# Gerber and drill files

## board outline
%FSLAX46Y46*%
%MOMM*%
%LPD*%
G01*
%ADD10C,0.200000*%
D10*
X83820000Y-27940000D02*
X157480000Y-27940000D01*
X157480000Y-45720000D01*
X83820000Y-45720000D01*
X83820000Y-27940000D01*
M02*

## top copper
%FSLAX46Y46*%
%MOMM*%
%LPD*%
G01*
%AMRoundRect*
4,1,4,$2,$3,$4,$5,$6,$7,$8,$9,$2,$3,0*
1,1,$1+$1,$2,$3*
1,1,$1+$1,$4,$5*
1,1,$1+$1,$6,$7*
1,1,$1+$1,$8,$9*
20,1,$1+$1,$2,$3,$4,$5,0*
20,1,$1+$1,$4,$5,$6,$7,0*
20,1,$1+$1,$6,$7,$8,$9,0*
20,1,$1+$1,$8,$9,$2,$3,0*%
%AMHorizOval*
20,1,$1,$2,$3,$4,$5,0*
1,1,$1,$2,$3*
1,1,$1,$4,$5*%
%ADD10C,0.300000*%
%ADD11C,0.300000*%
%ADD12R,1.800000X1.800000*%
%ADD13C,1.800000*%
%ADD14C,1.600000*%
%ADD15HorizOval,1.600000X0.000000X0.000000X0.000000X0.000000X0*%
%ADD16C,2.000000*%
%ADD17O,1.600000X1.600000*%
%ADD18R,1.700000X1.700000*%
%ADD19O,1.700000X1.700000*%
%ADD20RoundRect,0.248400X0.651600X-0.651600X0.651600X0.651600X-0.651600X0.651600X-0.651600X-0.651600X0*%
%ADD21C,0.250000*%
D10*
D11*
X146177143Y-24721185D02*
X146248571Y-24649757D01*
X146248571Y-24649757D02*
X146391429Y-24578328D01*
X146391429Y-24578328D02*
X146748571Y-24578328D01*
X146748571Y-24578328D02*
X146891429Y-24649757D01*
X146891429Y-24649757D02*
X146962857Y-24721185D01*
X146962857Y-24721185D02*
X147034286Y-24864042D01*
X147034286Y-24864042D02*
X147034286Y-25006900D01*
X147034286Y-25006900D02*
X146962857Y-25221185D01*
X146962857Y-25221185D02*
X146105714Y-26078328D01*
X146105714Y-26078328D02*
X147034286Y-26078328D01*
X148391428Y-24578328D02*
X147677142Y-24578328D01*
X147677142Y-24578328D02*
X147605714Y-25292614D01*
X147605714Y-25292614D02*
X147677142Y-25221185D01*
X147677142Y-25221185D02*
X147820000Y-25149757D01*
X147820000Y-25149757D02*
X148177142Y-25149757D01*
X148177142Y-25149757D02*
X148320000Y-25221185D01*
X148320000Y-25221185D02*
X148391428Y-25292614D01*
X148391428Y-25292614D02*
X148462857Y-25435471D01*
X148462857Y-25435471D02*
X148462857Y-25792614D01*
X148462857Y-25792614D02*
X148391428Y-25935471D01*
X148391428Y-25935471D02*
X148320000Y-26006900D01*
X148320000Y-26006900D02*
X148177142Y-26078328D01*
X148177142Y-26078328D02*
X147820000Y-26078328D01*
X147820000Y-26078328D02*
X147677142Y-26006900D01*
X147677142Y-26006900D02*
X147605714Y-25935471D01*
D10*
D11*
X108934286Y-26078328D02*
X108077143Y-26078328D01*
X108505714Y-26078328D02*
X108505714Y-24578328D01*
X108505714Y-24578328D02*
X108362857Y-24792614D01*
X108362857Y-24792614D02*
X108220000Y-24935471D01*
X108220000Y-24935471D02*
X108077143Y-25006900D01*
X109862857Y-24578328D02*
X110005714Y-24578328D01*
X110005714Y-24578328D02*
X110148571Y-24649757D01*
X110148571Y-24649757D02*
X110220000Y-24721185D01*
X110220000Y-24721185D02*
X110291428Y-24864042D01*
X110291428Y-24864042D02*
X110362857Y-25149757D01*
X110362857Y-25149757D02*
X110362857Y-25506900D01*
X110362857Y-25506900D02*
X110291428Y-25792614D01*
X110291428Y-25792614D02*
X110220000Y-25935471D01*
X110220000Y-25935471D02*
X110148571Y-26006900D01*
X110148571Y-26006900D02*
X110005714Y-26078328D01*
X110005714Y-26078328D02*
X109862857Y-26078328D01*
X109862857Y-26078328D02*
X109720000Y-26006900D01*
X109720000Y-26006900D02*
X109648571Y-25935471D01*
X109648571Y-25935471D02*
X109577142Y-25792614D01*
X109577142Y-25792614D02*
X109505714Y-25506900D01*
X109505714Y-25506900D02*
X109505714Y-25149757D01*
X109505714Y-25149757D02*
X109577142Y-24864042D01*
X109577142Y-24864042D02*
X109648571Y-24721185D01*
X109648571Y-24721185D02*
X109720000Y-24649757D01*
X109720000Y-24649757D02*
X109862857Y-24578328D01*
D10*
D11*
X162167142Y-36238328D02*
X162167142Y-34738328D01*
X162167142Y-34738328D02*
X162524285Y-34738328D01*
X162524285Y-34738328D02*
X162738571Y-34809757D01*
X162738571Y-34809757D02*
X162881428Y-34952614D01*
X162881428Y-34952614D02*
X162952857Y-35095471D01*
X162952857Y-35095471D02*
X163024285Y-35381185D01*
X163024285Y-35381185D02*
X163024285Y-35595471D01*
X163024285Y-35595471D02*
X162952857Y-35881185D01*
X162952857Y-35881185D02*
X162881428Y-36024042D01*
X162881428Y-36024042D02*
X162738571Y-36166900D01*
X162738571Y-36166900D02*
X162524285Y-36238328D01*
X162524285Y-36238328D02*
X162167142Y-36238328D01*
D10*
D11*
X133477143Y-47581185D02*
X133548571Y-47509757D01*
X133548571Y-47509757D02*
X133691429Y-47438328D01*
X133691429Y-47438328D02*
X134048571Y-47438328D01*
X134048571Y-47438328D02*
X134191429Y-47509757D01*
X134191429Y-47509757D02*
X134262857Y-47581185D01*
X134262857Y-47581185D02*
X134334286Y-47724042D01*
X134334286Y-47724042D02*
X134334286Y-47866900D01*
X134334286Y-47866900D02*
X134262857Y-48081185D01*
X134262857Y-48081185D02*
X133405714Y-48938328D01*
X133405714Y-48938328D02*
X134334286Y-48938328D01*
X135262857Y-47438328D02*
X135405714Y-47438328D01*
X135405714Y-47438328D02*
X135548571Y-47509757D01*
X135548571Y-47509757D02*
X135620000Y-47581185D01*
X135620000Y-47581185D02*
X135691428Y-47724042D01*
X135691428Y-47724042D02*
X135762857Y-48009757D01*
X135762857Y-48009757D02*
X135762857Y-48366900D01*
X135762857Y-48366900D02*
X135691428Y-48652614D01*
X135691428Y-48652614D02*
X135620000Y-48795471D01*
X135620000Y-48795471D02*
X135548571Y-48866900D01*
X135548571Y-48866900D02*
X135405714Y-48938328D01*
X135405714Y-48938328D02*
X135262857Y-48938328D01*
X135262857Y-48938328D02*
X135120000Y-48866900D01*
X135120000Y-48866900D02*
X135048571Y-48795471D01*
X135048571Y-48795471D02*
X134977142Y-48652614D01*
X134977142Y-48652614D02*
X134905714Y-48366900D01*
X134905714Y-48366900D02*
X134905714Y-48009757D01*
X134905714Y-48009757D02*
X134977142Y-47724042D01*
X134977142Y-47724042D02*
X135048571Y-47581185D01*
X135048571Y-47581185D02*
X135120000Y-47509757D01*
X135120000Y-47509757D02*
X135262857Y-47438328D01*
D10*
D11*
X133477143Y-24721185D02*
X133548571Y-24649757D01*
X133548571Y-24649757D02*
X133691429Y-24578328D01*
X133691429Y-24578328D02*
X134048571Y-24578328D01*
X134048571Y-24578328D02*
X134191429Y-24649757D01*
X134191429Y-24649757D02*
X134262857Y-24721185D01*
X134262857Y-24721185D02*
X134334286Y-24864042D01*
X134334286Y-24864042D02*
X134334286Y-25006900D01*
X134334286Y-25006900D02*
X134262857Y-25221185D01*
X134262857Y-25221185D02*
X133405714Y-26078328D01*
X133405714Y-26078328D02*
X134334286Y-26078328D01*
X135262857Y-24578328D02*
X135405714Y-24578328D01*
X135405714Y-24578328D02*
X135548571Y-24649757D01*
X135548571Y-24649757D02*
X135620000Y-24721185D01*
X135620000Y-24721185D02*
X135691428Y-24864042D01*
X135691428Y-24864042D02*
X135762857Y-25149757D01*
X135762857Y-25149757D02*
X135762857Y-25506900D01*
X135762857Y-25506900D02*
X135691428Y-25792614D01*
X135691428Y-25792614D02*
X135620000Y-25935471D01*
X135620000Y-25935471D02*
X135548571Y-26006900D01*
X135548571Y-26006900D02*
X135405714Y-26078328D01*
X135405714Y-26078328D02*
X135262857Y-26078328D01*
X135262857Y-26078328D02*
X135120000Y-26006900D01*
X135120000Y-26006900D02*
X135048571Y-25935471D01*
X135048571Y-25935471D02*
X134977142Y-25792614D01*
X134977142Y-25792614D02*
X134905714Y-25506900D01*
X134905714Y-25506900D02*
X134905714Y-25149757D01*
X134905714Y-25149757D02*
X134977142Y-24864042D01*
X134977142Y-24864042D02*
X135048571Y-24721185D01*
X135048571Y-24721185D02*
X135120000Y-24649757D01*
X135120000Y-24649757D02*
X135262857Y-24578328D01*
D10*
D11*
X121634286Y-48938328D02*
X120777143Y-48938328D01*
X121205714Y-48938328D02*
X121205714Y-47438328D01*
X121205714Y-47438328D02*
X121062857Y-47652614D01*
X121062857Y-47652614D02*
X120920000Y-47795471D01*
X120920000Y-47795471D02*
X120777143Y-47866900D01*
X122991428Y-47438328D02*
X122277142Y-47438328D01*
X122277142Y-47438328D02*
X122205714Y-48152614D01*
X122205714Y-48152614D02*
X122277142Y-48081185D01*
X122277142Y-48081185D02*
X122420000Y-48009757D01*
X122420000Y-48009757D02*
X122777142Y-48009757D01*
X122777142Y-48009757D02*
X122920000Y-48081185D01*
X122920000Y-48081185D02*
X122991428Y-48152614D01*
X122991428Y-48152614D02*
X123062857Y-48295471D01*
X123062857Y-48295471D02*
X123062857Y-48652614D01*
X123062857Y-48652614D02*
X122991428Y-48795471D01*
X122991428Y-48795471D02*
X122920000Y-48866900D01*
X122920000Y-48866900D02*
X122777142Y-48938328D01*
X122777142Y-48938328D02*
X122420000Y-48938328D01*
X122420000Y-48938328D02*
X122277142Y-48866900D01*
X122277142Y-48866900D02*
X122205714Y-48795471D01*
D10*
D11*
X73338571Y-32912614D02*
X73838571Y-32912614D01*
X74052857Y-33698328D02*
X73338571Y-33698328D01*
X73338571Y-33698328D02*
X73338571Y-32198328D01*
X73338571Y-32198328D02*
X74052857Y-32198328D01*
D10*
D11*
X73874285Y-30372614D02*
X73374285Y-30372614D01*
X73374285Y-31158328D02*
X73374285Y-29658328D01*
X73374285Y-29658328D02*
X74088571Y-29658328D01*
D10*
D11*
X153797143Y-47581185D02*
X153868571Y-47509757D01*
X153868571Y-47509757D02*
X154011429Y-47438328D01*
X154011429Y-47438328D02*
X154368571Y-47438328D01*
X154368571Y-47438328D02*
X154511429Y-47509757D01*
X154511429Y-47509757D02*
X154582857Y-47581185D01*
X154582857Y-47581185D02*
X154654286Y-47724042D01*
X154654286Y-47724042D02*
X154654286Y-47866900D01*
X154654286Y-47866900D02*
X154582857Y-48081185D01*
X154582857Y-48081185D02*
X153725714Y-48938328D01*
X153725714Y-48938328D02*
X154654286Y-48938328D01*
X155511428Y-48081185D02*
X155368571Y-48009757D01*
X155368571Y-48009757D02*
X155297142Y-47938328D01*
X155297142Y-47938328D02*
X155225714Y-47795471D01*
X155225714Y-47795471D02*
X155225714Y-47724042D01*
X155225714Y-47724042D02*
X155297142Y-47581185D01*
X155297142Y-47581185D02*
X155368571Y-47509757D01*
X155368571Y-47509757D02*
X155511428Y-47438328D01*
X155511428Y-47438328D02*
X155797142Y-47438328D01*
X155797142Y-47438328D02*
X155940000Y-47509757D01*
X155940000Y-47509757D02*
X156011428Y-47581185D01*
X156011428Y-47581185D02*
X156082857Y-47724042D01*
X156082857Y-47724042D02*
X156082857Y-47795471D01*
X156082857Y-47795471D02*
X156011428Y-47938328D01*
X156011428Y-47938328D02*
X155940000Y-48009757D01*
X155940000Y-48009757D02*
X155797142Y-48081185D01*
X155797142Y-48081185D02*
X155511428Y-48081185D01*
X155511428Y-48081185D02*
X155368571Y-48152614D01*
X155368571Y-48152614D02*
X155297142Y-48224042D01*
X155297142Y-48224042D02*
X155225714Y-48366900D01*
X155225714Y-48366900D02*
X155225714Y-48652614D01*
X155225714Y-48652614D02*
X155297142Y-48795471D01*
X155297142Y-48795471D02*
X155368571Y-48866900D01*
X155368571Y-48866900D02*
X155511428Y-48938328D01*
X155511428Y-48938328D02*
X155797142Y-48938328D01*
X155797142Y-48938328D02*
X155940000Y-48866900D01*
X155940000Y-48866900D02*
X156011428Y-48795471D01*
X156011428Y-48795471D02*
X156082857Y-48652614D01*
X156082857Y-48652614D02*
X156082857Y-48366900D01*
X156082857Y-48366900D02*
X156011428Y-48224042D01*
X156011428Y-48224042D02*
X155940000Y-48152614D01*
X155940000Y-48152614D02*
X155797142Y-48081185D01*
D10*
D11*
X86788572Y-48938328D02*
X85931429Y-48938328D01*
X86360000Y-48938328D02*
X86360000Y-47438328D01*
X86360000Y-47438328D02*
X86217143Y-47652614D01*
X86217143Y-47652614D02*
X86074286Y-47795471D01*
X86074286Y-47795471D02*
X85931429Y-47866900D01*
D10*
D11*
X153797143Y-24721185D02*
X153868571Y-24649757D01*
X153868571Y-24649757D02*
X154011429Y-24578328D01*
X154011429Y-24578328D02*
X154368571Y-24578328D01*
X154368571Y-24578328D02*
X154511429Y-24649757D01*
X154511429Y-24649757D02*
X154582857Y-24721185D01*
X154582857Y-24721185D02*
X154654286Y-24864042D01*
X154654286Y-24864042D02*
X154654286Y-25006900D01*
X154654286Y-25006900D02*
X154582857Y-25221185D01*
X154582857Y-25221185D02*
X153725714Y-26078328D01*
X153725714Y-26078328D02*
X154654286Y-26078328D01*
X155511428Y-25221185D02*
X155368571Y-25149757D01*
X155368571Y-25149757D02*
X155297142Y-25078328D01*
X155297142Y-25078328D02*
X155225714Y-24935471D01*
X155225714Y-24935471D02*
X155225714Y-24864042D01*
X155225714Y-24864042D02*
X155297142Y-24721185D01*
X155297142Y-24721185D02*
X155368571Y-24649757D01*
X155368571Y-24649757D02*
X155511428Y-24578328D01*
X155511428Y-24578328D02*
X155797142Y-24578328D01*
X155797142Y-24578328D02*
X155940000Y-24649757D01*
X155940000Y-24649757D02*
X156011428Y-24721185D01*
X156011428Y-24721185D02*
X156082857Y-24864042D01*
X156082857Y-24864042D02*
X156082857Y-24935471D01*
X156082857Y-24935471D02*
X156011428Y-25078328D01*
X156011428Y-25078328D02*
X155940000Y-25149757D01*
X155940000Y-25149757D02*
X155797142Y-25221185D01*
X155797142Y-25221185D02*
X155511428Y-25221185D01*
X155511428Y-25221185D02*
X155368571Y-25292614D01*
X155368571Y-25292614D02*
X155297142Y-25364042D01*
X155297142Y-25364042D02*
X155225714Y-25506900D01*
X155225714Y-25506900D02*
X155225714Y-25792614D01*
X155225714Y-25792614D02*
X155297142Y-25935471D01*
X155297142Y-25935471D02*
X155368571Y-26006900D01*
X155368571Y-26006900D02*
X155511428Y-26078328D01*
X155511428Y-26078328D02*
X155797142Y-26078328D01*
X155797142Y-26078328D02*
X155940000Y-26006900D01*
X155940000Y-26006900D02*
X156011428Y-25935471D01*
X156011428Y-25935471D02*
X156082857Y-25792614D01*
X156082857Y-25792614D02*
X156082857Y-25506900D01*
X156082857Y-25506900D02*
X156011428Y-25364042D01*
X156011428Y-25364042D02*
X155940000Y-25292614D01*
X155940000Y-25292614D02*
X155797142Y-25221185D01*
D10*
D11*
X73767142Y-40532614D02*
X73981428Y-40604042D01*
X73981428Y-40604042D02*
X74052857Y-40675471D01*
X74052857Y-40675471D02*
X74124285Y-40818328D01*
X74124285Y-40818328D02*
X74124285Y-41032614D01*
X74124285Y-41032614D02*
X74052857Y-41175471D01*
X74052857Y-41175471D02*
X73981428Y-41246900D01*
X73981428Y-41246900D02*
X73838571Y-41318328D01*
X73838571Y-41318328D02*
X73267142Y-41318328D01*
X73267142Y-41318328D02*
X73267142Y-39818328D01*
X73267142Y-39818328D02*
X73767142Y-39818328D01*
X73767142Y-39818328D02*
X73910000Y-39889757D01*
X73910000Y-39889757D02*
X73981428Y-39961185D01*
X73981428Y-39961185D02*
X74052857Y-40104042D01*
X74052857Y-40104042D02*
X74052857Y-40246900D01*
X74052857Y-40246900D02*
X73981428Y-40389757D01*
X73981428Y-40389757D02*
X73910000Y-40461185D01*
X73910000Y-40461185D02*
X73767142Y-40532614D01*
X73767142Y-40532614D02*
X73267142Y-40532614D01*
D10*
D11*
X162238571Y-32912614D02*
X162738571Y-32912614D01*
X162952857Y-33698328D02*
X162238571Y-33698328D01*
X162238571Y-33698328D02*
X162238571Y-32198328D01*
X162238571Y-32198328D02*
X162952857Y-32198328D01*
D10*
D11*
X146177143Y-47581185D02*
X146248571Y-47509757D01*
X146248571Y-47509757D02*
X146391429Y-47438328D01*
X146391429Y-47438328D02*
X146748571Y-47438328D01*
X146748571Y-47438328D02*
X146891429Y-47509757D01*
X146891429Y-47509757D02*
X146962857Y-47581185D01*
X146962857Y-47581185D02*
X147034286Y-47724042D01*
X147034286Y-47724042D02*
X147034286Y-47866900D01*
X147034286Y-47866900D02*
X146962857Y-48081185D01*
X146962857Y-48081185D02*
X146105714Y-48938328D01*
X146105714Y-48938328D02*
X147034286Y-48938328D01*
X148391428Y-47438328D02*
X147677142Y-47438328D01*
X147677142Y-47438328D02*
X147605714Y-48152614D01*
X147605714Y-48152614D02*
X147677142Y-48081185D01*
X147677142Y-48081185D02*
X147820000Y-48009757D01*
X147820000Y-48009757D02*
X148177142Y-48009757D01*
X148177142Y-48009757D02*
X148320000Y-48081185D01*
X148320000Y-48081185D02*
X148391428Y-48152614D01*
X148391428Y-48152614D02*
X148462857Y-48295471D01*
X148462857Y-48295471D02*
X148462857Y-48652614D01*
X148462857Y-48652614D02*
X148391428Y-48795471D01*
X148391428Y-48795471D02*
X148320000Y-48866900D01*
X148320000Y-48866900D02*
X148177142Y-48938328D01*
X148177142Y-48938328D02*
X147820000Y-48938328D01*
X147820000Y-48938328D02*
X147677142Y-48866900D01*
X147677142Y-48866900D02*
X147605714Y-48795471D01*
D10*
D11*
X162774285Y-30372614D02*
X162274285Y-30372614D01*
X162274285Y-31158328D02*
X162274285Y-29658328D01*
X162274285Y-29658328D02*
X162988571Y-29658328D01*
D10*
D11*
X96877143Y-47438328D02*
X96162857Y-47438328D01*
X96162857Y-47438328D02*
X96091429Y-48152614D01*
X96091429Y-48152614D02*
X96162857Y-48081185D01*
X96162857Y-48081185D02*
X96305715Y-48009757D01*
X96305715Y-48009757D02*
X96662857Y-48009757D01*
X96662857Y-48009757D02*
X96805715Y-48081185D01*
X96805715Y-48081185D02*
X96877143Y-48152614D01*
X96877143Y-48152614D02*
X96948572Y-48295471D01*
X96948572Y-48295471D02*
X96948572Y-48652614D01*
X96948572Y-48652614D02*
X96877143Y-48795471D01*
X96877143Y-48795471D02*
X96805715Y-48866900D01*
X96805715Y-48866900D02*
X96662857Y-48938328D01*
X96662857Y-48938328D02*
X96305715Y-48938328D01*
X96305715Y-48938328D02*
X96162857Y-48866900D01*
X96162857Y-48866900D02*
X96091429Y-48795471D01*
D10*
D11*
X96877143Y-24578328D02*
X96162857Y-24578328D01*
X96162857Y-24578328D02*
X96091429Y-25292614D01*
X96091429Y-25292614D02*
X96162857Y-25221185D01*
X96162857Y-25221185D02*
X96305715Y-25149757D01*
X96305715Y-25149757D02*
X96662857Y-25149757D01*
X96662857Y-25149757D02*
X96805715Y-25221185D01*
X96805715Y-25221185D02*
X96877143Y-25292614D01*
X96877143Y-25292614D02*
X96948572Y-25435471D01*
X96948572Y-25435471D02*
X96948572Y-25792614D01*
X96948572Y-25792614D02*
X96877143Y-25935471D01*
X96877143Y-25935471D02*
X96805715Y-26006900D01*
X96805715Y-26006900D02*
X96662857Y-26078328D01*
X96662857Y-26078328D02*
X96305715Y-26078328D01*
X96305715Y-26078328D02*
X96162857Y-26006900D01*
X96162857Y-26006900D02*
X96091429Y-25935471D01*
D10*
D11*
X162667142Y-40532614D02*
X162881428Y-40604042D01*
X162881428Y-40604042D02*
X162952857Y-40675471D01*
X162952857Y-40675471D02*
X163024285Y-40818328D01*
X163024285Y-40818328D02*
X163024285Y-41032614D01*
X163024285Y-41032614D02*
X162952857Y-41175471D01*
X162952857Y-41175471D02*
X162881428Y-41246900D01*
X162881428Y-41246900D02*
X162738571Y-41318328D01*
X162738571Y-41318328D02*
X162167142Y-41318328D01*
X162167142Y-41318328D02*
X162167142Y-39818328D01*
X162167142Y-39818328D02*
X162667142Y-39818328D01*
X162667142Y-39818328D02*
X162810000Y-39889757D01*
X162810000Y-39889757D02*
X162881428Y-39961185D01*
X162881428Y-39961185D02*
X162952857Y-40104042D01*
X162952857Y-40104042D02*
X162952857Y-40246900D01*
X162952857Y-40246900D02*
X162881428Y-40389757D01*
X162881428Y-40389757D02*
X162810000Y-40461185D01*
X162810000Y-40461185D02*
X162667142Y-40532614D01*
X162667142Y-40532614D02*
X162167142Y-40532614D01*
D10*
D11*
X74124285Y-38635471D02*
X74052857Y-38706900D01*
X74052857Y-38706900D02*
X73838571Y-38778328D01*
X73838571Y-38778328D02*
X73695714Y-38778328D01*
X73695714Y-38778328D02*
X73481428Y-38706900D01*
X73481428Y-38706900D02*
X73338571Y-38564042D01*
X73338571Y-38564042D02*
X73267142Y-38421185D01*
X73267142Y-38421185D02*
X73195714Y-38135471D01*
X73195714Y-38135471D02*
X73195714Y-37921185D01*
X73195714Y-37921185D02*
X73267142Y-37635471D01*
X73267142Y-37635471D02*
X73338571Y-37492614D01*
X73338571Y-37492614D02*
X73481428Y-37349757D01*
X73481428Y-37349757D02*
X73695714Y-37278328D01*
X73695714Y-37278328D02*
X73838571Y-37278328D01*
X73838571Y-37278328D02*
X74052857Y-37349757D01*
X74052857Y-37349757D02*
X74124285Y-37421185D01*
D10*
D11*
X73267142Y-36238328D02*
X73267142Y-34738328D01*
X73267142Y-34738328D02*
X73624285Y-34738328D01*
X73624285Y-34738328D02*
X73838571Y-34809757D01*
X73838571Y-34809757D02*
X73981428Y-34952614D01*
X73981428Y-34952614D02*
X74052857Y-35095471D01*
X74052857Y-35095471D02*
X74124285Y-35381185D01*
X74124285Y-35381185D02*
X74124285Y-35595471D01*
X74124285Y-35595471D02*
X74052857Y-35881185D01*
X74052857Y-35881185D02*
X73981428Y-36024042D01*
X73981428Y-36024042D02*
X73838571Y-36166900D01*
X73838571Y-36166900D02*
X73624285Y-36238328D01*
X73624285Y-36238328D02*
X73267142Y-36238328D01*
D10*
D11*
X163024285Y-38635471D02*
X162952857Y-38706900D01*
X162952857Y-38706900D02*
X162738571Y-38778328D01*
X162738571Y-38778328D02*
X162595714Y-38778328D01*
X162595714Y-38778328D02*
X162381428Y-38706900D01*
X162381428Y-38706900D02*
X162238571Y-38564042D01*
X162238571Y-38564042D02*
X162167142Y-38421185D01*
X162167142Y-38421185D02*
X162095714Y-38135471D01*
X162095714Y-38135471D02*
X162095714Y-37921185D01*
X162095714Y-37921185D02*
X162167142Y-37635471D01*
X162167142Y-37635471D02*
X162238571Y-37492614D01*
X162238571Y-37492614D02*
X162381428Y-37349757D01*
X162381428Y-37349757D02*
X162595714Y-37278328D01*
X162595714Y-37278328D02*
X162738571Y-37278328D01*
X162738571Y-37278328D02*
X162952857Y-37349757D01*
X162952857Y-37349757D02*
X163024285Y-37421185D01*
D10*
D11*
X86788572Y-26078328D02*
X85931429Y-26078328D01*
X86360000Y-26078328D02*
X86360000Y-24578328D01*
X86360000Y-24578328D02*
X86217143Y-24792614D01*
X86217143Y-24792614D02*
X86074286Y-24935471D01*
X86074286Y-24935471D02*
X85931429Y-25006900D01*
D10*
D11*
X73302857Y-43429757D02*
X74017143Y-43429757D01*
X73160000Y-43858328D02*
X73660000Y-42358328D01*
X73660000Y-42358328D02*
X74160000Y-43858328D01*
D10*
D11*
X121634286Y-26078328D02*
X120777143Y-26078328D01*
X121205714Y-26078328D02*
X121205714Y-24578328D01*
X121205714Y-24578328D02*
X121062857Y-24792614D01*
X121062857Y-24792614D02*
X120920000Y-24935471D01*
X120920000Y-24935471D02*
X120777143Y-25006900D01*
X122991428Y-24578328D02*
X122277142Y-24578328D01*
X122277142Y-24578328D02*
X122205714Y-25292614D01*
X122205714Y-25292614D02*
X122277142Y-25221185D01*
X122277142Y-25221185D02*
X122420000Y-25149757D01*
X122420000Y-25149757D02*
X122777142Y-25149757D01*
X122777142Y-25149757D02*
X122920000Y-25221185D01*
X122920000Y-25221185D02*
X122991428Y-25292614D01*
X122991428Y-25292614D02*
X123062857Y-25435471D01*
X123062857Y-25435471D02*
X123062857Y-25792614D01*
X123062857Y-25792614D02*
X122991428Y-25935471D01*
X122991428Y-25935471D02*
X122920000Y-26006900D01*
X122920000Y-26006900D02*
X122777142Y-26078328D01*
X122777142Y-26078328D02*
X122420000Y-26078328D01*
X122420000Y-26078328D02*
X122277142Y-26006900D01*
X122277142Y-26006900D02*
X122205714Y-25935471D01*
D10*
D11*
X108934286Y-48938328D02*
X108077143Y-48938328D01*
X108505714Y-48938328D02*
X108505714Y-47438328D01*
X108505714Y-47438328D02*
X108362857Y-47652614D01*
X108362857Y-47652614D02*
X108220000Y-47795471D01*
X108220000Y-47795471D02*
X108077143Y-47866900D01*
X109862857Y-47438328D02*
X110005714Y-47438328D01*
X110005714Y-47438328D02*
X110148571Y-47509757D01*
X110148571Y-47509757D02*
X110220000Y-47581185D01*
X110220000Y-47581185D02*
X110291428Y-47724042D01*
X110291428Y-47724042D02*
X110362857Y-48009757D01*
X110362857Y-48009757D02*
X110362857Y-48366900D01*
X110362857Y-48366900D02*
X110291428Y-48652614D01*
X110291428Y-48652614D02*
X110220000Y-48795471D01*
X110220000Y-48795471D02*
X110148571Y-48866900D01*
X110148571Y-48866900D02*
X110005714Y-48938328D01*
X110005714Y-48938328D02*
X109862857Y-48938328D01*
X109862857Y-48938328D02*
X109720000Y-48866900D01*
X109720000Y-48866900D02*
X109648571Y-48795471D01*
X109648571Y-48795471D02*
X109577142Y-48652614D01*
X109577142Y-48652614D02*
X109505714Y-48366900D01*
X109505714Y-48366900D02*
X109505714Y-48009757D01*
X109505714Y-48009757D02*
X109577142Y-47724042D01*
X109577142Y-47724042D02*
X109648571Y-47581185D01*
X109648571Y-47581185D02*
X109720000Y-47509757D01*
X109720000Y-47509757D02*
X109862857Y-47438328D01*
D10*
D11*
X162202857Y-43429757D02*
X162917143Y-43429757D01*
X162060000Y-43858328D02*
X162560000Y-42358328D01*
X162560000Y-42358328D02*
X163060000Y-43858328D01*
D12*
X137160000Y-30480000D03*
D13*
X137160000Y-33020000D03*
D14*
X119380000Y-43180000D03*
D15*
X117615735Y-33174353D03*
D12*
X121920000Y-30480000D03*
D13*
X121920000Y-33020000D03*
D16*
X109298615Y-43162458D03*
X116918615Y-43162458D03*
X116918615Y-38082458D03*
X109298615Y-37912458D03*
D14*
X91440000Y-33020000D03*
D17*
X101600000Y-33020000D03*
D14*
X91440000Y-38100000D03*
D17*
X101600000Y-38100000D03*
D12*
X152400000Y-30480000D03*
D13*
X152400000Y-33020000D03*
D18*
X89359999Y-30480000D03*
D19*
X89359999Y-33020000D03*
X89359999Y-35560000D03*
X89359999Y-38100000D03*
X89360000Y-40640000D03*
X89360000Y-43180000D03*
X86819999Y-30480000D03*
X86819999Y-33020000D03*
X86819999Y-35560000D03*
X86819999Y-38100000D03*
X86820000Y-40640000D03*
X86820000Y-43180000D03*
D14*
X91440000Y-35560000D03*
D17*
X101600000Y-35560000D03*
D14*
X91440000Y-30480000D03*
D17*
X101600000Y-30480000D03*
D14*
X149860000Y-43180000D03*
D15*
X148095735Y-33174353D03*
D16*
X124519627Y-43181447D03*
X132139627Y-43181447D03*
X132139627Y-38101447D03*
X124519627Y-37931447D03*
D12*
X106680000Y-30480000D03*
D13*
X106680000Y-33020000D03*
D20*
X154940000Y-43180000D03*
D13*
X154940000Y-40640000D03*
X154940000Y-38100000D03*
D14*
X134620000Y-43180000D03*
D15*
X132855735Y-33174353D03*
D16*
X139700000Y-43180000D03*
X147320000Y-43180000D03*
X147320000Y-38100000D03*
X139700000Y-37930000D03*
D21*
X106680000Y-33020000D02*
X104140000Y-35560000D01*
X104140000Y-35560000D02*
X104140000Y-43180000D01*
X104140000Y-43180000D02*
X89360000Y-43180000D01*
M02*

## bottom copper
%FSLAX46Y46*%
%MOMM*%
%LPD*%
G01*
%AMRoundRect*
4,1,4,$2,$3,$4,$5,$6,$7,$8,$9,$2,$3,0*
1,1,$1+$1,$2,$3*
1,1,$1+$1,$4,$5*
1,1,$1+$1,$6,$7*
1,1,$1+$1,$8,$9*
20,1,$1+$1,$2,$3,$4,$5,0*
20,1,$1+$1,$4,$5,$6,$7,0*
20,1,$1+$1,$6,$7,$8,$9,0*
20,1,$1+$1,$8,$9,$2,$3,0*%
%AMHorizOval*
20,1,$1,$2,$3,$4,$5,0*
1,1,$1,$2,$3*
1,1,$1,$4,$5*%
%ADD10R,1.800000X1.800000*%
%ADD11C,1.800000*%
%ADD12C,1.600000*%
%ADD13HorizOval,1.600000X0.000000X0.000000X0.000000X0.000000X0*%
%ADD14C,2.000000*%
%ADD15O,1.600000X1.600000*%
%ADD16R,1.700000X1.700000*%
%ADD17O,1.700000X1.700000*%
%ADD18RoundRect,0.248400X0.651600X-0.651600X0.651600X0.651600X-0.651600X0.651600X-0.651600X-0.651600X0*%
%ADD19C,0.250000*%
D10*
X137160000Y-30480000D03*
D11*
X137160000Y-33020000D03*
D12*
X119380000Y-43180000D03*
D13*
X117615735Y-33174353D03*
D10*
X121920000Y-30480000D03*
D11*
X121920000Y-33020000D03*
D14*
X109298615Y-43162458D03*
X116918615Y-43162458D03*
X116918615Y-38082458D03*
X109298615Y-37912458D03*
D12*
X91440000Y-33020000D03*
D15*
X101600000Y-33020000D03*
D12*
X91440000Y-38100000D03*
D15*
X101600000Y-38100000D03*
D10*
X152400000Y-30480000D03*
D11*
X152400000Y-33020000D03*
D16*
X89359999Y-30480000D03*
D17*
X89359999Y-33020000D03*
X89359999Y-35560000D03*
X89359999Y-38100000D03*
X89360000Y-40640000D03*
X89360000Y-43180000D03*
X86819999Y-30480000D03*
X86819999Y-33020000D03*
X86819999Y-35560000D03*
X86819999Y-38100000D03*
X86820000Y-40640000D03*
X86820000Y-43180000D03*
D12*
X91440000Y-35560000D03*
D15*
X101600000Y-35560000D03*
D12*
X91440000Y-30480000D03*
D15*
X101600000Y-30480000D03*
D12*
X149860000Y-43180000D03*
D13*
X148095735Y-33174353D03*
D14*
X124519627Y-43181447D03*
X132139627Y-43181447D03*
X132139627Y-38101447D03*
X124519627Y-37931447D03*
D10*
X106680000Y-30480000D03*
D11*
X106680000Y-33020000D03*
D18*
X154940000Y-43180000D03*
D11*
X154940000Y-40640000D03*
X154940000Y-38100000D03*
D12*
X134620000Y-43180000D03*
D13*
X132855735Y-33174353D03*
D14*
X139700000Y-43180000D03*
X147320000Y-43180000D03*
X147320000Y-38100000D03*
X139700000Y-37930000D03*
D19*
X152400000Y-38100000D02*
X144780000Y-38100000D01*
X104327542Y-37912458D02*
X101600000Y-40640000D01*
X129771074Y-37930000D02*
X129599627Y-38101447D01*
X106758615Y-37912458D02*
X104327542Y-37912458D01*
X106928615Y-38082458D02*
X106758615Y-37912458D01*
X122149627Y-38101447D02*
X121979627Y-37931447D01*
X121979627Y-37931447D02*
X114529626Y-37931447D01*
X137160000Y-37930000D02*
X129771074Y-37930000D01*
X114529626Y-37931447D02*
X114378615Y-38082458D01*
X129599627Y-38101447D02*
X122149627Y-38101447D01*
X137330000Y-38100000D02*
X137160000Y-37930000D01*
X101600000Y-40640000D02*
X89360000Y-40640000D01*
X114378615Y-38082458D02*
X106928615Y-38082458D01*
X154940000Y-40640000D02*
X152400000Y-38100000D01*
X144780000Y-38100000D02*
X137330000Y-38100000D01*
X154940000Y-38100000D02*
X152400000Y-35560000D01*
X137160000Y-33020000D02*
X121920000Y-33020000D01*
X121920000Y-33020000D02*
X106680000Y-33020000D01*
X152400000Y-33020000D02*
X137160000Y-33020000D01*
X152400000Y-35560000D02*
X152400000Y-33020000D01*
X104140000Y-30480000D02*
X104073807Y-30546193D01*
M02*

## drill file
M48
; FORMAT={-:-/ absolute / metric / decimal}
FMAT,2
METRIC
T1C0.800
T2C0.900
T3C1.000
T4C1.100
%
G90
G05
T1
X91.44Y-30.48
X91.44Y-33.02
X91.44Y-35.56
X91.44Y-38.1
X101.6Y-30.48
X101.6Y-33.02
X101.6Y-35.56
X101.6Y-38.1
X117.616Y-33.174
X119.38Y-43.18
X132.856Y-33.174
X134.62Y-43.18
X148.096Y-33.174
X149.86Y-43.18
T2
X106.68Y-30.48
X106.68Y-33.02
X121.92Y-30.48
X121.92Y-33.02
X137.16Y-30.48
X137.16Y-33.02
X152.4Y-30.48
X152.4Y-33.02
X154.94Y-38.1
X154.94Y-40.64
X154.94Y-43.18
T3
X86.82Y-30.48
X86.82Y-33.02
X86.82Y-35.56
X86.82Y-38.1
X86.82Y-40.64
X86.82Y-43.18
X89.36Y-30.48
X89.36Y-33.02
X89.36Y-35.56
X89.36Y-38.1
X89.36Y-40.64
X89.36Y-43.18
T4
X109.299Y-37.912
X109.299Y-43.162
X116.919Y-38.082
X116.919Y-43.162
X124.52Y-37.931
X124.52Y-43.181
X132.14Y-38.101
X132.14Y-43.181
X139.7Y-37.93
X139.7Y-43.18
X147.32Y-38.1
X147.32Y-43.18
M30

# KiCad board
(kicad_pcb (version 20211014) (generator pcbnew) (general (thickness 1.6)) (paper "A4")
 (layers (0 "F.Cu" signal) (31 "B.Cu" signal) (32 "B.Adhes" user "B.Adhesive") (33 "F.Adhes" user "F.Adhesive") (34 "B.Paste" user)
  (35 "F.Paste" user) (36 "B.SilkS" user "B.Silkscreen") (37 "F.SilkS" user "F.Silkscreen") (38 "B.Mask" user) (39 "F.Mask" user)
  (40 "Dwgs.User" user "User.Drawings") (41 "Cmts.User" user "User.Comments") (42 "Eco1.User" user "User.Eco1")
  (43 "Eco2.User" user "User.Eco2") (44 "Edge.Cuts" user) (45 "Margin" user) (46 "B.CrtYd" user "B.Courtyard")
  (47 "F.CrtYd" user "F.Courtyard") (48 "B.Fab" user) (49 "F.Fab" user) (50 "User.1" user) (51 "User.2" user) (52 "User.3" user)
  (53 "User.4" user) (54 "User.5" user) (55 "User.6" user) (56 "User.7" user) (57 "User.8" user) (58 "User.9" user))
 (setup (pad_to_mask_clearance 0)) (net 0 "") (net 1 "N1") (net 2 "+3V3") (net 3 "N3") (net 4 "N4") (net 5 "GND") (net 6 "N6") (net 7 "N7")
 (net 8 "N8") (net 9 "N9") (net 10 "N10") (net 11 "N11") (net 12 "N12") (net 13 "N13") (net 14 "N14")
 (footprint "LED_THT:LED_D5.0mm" (layer "F.Cu") (at 137.16 30.48 -90)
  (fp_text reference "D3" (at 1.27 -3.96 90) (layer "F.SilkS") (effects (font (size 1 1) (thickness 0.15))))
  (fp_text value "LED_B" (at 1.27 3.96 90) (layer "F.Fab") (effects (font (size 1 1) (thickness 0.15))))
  (pad "1" thru_hole rect (at 0 0 270) (size 1.8 1.8) (drill 0.9) (layers *.Cu *.Mask) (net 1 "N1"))
  (pad "2" thru_hole circle (at 2.54 0 270) (size 1.8 1.8) (drill 0.9) (layers *.Cu *.Mask) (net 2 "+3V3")))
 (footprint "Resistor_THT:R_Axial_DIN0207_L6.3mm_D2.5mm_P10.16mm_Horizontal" (layer "F.Cu") (at 119.38 43.18 100)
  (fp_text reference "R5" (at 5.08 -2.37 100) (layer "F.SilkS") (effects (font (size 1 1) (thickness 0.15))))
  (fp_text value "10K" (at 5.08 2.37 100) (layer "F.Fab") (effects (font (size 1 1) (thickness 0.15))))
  (pad "1" thru_hole circle (at 0 0 100) (size 1.6 1.6) (drill 0.8) (layers *.Cu *.Mask) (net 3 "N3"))
  (pad "2" thru_hole oval (at 10.16 0 100) (size 1.6 1.6) (drill 0.8) (layers *.Cu *.Mask) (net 2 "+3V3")))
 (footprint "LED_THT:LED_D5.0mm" (layer "F.Cu") (at 121.92 30.48 -90)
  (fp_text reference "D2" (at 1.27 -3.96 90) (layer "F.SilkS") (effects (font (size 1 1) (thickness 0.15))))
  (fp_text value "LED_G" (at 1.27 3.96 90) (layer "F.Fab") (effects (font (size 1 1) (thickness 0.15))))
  (pad "1" thru_hole rect (at 0 0 270) (size 1.8 1.8) (drill 0.9) (layers *.Cu *.Mask) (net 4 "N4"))
  (pad "2" thru_hole circle (at 2.54 0 270) (size 1.8 1.8) (drill 0.9) (layers *.Cu *.Mask) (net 2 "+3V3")))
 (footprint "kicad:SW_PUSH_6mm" (layer "F.Cu") (at 116.918615 43.162458 180)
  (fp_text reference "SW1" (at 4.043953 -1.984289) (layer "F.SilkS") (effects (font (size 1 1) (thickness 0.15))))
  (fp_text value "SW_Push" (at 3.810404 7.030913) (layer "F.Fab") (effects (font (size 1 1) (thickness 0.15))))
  (pad "1" thru_hole circle (at 7.62 0 270) (size 2 2) (drill 1.1) (layers *.Cu *.Mask) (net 3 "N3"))
  (pad "1" thru_hole circle (at 0 0 270) (size 2 2) (drill 1.1) (layers *.Cu *.Mask) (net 3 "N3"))
  (pad "2" thru_hole circle (at 0 5.08 270) (size 2 2) (drill 1.1) (layers *.Cu *.Mask) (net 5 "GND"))
  (pad "2" thru_hole circle (at 7.62 5.25 270) (size 2 2) (drill 1.1) (layers *.Cu *.Mask) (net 5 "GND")))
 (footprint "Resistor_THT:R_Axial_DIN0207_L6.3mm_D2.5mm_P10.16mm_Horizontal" (layer "F.Cu") (at 91.44 33.02)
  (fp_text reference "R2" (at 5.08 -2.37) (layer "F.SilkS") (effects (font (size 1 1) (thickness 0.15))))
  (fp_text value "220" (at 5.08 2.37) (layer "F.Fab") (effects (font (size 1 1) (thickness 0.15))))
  (pad "1" thru_hole circle (at 0 0) (size 1.6 1.6) (drill 0.8) (layers *.Cu *.Mask) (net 4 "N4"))
  (pad "2" thru_hole oval (at 10.16 0) (size 1.6 1.6) (drill 0.8) (layers *.Cu *.Mask) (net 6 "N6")))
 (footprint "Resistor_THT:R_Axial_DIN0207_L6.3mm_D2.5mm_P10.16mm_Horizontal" (layer "F.Cu") (at 91.44 38.1)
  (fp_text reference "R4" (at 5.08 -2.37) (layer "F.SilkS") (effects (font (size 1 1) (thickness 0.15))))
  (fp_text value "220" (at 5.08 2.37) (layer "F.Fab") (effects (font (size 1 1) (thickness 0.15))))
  (pad "1" thru_hole circle (at 0 0) (size 1.6 1.6) (drill 0.8) (layers *.Cu *.Mask) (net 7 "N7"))
  (pad "2" thru_hole oval (at 10.16 0) (size 1.6 1.6) (drill 0.8) (layers *.Cu *.Mask) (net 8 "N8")))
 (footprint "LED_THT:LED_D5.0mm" (layer "F.Cu") (at 152.4 30.48 -90)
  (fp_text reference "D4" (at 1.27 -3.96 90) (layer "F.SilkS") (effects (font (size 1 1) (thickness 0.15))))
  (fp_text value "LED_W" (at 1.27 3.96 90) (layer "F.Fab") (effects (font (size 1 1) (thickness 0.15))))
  (pad "1" thru_hole rect (at 0 0 270) (size 1.8 1.8) (drill 0.9) (layers *.Cu *.Mask) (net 7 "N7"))
  (pad "2" thru_hole circle (at 2.54 0 270) (size 1.8 1.8) (drill 0.9) (layers *.Cu *.Mask) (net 2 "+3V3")))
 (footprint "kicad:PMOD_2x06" (layer "F.Cu") (at 78.74 30.48)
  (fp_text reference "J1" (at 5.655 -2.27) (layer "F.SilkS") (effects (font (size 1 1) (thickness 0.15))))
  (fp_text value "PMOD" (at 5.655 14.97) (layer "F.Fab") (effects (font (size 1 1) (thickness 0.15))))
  (pad "a1" thru_hole rect (at 10.619999 0) (size 1.7 1.7) (drill 1) (layers *.Cu *.Mask) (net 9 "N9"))
  (pad "a2" thru_hole oval (at 10.619999 2.54) (size 1.7 1.7) (drill 1) (layers *.Cu *.Mask) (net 6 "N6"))
  (pad "a3" thru_hole oval (at 10.619999 5.08) (size 1.7 1.7) (drill 1) (layers *.Cu *.Mask) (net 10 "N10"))
  (pad "a4" thru_hole oval (at 10.619999 7.62) (size 1.7 1.7) (drill 1) (layers *.Cu *.Mask) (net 8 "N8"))
  (pad "a5" thru_hole oval (at 10.62 10.16) (size 1.7 1.7) (drill 1) (layers *.Cu *.Mask) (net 5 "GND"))
  (pad "a6" thru_hole oval (at 10.62 12.7) (size 1.7 1.7) (drill 1) (layers *.Cu *.Mask) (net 2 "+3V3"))
  (pad "b1" thru_hole oval (at 8.079999 0) (size 1.7 1.7) (drill 1) (layers *.Cu *.Mask) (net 3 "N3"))
  (pad "b2" thru_hole oval (at 8.079999 2.54) (size 1.7 1.7) (drill 1) (layers *.Cu *.Mask) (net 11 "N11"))
  (pad "b3" thru_hole oval (at 8.079999 5.08) (size 1.7 1.7) (drill 1) (layers *.Cu *.Mask) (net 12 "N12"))
  (pad "b4" thru_hole oval (at 8.079999 7.62) (size 1.7 1.7) (drill 1) (layers *.Cu *.Mask) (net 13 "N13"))
  (pad "b5" thru_hole oval (at 8.08 10.16) (size 1.7 1.7) (drill 1) (layers *.Cu *.Mask) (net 5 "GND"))
  (pad "b6" thru_hole oval (at 8.08 12.7) (size 1.7 1.7) (drill 1) (layers *.Cu *.Mask) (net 2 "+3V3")))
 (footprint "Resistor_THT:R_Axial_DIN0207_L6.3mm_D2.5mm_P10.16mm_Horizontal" (layer "F.Cu") (at 91.44 35.56)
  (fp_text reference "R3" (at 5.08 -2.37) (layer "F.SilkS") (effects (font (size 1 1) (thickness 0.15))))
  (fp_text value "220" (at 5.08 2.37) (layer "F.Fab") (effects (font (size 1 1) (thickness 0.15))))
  (pad "1" thru_hole circle (at 0 0) (size 1.6 1.6) (drill 0.8) (layers *.Cu *.Mask) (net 1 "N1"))
  (pad "2" thru_hole oval (at 10.16 0) (size 1.6 1.6) (drill 0.8) (layers *.Cu *.Mask) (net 10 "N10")))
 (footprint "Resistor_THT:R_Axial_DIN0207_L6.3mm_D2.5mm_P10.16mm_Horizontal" (layer "F.Cu") (at 91.44 30.48)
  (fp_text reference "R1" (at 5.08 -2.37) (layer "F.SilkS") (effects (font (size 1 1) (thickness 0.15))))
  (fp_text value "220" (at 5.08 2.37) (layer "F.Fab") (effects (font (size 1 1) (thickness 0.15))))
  (pad "1" thru_hole circle (at 0 0) (size 1.6 1.6) (drill 0.8) (layers *.Cu *.Mask) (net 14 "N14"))
  (pad "2" thru_hole oval (at 10.16 0) (size 1.6 1.6) (drill 0.8) (layers *.Cu *.Mask) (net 9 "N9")))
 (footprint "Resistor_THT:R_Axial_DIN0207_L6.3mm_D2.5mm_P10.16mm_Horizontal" (layer "F.Cu") (at 149.86 43.18 100)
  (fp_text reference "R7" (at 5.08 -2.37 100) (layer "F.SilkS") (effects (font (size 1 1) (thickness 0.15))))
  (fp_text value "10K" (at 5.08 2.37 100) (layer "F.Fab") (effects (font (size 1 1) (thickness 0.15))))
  (pad "1" thru_hole circle (at 0 0 100) (size 1.6 1.6) (drill 0.8) (layers *.Cu *.Mask) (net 12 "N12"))
  (pad "2" thru_hole oval (at 10.16 0 100) (size 1.6 1.6) (drill 0.8) (layers *.Cu *.Mask) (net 2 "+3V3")))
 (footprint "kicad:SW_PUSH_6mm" (layer "F.Cu") (at 132.139627 43.181447 180)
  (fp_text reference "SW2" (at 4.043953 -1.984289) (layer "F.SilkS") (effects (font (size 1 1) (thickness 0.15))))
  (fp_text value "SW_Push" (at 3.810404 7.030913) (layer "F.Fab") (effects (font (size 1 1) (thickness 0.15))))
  (pad "1" thru_hole circle (at 7.62 0 270) (size 2 2) (drill 1.1) (layers *.Cu *.Mask) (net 11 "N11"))
  (pad "1" thru_hole circle (at 0 0 270) (size 2 2) (drill 1.1) (layers *.Cu *.Mask) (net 11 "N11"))
  (pad "2" thru_hole circle (at 0 5.08 270) (size 2 2) (drill 1.1) (layers *.Cu *.Mask) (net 5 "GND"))
  (pad "2" thru_hole circle (at 7.62 5.25 270) (size 2 2) (drill 1.1) (layers *.Cu *.Mask) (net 5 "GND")))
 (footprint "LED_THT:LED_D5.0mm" (layer "F.Cu") (at 106.68 30.48 -90)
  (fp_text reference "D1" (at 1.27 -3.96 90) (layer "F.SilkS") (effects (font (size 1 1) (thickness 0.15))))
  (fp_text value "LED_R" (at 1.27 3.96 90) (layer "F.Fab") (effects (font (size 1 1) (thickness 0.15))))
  (pad "1" thru_hole rect (at 0 0 270) (size 1.8 1.8) (drill 0.9) (layers *.Cu *.Mask) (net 14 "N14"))
  (pad "2" thru_hole circle (at 2.54 0 270) (size 1.8 1.8) (drill 0.9) (layers *.Cu *.Mask) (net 2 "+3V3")))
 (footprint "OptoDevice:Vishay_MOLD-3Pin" (layer "F.Cu") (at 154.94 43.18 90)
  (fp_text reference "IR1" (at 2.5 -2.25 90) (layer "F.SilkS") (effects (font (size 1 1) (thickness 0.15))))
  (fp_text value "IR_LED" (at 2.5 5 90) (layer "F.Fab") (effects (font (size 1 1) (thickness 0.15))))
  (pad "1" thru_hole roundrect (at 0 0 90) (size 1.8 1.8) (drill 0.9) (layers *.Cu *.Mask) (roundrect_rratio 0.138) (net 13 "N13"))
  (pad "2" thru_hole circle (at 2.54 0 90) (size 1.8 1.8) (drill 0.9) (layers *.Cu *.Mask) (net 5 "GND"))
  (pad "3" thru_hole circle (at 5.08 0 90) (size 1.8 1.8) (drill 0.9) (layers *.Cu *.Mask) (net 2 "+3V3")))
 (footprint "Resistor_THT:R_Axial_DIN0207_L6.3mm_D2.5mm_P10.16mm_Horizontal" (layer "F.Cu") (at 134.62 43.18 100)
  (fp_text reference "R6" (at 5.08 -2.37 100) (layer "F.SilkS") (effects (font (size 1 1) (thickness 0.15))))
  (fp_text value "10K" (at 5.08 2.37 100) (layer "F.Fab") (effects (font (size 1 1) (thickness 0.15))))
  (pad "1" thru_hole circle (at 0 0 100) (size 1.6 1.6) (drill 0.8) (layers *.Cu *.Mask) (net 11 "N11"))
  (pad "2" thru_hole oval (at 10.16 0 100) (size 1.6 1.6) (drill 0.8) (layers *.Cu *.Mask) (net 2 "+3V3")))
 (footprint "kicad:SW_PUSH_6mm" (layer "F.Cu") (at 147.32 43.18 180)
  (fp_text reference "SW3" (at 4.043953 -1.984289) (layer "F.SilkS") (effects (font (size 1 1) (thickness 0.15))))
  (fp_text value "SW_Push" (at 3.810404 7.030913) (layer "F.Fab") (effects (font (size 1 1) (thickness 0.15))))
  (pad "1" thru_hole circle (at 7.62 0 270) (size 2 2) (drill 1.1) (layers *.Cu *.Mask) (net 12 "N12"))
  (pad "1" thru_hole circle (at 0 0 270) (size 2 2) (drill 1.1) (layers *.Cu *.Mask) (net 12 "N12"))
  (pad "2" thru_hole circle (at 0 5.08 270) (size 2 2) (drill 1.1) (layers *.Cu *.Mask) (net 5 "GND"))
  (pad "2" thru_hole circle (at 7.62 5.25 270) (size 2 2) (drill 1.1) (layers *.Cu *.Mask) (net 5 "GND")))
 (gr_rect (start 83.82 27.94) (end 157.48 45.72) (layer "Edge.Cuts") (width 0.2) (fill none))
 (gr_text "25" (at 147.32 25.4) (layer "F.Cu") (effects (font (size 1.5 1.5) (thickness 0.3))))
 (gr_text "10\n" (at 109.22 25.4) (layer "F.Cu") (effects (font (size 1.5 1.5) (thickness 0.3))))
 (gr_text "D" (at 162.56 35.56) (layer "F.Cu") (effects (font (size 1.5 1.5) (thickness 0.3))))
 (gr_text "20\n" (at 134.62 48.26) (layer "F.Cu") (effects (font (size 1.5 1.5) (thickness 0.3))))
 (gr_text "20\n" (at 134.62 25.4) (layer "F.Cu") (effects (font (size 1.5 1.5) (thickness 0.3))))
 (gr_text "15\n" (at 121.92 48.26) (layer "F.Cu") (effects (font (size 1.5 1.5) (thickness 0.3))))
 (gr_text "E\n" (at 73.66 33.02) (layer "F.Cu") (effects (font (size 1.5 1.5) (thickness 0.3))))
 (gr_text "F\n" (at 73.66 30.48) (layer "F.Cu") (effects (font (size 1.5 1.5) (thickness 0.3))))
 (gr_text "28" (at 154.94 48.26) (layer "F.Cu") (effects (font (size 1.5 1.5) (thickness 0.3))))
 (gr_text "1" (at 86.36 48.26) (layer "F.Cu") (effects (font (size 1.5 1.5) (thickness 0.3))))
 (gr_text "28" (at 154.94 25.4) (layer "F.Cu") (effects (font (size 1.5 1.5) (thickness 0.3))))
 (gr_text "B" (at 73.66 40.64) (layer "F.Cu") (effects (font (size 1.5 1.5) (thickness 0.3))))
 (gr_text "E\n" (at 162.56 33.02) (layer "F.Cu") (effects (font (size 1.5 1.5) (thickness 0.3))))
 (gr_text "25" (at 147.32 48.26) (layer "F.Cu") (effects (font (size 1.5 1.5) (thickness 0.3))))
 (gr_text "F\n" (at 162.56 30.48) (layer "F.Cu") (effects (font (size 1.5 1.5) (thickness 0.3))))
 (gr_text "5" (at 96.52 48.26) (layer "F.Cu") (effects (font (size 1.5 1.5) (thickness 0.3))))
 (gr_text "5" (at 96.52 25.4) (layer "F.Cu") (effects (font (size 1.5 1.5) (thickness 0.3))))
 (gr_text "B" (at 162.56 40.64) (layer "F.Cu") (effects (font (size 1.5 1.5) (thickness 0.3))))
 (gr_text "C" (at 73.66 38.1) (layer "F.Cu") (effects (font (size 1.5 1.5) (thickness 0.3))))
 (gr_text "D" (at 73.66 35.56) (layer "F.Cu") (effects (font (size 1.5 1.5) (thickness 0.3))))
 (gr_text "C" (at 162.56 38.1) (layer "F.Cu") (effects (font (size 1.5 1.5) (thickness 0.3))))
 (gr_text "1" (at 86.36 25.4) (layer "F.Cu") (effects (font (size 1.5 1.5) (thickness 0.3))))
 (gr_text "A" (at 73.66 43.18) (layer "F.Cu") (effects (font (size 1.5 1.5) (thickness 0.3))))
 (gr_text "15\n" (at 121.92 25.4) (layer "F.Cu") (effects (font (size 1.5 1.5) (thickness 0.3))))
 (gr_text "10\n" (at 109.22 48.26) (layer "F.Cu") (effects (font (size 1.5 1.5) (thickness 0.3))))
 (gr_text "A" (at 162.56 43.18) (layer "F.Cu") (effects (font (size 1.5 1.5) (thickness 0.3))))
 (segment (start 152.4 38.1) (end 144.78 38.1) (width 0.25) (layer "B.Cu") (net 5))
 (segment (start 104.327542 37.912458) (end 101.6 40.64) (width 0.25) (layer "B.Cu") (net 5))
 (segment (start 129.771074 37.93) (end 129.599627 38.101447) (width 0.25) (layer "B.Cu") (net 5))
 (segment (start 106.758615 37.912458) (end 104.327542 37.912458) (width 0.25) (layer "B.Cu") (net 5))
 (segment (start 106.928615 38.082458) (end 106.758615 37.912458) (width 0.25) (layer "B.Cu") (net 5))
 (segment (start 122.149627 38.101447) (end 121.979627 37.931447) (width 0.25) (layer "B.Cu") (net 5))
 (segment (start 121.979627 37.931447) (end 114.529626 37.931447) (width 0.25) (layer "B.Cu") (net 5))
 (segment (start 137.16 37.93) (end 129.771074 37.93) (width 0.25) (layer "B.Cu") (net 5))
 (segment (start 114.529626 37.931447) (end 114.378615 38.082458) (width 0.25) (layer "B.Cu") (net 5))
 (segment (start 129.599627 38.101447) (end 122.149627 38.101447) (width 0.25) (layer "B.Cu") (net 5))
 (segment (start 137.33 38.1) (end 137.16 37.93) (width 0.25) (layer "B.Cu") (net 5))
 (segment (start 101.6 40.64) (end 89.36 40.64) (width 0.25) (layer "B.Cu") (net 5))
 (segment (start 114.378615 38.082458) (end 106.928615 38.082458) (width 0.25) (layer "B.Cu") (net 5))
 (segment (start 154.94 40.64) (end 152.4 38.1) (width 0.25) (layer "B.Cu") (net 5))
 (segment (start 144.78 38.1) (end 137.33 38.1) (width 0.25) (layer "B.Cu") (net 5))
 (segment (start 106.68 33.02) (end 104.14 35.56) (width 0.25) (layer "F.Cu") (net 2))
 (segment (start 104.14 35.56) (end 104.14 43.18) (width 0.25) (layer "F.Cu") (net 2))
 (segment (start 104.14 43.18) (end 89.36 43.18) (width 0.25) (layer "F.Cu") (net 2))
 (segment (start 154.94 38.1) (end 152.4 35.56) (width 0.25) (layer "B.Cu") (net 2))
 (segment (start 137.16 33.02) (end 121.92 33.02) (width 0.25) (layer "B.Cu") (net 2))
 (segment (start 121.92 33.02) (end 106.68 33.02) (width 0.25) (layer "B.Cu") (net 2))
 (segment (start 152.4 33.02) (end 137.16 33.02) (width 0.25) (layer "B.Cu") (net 2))
 (segment (start 152.4 35.56) (end 152.4 33.02) (width 0.25) (layer "B.Cu") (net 2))
 (segment (start 104.14 30.48) (end 104.073807 30.546193) (width 0.25) (layer "B.Cu") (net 14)))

